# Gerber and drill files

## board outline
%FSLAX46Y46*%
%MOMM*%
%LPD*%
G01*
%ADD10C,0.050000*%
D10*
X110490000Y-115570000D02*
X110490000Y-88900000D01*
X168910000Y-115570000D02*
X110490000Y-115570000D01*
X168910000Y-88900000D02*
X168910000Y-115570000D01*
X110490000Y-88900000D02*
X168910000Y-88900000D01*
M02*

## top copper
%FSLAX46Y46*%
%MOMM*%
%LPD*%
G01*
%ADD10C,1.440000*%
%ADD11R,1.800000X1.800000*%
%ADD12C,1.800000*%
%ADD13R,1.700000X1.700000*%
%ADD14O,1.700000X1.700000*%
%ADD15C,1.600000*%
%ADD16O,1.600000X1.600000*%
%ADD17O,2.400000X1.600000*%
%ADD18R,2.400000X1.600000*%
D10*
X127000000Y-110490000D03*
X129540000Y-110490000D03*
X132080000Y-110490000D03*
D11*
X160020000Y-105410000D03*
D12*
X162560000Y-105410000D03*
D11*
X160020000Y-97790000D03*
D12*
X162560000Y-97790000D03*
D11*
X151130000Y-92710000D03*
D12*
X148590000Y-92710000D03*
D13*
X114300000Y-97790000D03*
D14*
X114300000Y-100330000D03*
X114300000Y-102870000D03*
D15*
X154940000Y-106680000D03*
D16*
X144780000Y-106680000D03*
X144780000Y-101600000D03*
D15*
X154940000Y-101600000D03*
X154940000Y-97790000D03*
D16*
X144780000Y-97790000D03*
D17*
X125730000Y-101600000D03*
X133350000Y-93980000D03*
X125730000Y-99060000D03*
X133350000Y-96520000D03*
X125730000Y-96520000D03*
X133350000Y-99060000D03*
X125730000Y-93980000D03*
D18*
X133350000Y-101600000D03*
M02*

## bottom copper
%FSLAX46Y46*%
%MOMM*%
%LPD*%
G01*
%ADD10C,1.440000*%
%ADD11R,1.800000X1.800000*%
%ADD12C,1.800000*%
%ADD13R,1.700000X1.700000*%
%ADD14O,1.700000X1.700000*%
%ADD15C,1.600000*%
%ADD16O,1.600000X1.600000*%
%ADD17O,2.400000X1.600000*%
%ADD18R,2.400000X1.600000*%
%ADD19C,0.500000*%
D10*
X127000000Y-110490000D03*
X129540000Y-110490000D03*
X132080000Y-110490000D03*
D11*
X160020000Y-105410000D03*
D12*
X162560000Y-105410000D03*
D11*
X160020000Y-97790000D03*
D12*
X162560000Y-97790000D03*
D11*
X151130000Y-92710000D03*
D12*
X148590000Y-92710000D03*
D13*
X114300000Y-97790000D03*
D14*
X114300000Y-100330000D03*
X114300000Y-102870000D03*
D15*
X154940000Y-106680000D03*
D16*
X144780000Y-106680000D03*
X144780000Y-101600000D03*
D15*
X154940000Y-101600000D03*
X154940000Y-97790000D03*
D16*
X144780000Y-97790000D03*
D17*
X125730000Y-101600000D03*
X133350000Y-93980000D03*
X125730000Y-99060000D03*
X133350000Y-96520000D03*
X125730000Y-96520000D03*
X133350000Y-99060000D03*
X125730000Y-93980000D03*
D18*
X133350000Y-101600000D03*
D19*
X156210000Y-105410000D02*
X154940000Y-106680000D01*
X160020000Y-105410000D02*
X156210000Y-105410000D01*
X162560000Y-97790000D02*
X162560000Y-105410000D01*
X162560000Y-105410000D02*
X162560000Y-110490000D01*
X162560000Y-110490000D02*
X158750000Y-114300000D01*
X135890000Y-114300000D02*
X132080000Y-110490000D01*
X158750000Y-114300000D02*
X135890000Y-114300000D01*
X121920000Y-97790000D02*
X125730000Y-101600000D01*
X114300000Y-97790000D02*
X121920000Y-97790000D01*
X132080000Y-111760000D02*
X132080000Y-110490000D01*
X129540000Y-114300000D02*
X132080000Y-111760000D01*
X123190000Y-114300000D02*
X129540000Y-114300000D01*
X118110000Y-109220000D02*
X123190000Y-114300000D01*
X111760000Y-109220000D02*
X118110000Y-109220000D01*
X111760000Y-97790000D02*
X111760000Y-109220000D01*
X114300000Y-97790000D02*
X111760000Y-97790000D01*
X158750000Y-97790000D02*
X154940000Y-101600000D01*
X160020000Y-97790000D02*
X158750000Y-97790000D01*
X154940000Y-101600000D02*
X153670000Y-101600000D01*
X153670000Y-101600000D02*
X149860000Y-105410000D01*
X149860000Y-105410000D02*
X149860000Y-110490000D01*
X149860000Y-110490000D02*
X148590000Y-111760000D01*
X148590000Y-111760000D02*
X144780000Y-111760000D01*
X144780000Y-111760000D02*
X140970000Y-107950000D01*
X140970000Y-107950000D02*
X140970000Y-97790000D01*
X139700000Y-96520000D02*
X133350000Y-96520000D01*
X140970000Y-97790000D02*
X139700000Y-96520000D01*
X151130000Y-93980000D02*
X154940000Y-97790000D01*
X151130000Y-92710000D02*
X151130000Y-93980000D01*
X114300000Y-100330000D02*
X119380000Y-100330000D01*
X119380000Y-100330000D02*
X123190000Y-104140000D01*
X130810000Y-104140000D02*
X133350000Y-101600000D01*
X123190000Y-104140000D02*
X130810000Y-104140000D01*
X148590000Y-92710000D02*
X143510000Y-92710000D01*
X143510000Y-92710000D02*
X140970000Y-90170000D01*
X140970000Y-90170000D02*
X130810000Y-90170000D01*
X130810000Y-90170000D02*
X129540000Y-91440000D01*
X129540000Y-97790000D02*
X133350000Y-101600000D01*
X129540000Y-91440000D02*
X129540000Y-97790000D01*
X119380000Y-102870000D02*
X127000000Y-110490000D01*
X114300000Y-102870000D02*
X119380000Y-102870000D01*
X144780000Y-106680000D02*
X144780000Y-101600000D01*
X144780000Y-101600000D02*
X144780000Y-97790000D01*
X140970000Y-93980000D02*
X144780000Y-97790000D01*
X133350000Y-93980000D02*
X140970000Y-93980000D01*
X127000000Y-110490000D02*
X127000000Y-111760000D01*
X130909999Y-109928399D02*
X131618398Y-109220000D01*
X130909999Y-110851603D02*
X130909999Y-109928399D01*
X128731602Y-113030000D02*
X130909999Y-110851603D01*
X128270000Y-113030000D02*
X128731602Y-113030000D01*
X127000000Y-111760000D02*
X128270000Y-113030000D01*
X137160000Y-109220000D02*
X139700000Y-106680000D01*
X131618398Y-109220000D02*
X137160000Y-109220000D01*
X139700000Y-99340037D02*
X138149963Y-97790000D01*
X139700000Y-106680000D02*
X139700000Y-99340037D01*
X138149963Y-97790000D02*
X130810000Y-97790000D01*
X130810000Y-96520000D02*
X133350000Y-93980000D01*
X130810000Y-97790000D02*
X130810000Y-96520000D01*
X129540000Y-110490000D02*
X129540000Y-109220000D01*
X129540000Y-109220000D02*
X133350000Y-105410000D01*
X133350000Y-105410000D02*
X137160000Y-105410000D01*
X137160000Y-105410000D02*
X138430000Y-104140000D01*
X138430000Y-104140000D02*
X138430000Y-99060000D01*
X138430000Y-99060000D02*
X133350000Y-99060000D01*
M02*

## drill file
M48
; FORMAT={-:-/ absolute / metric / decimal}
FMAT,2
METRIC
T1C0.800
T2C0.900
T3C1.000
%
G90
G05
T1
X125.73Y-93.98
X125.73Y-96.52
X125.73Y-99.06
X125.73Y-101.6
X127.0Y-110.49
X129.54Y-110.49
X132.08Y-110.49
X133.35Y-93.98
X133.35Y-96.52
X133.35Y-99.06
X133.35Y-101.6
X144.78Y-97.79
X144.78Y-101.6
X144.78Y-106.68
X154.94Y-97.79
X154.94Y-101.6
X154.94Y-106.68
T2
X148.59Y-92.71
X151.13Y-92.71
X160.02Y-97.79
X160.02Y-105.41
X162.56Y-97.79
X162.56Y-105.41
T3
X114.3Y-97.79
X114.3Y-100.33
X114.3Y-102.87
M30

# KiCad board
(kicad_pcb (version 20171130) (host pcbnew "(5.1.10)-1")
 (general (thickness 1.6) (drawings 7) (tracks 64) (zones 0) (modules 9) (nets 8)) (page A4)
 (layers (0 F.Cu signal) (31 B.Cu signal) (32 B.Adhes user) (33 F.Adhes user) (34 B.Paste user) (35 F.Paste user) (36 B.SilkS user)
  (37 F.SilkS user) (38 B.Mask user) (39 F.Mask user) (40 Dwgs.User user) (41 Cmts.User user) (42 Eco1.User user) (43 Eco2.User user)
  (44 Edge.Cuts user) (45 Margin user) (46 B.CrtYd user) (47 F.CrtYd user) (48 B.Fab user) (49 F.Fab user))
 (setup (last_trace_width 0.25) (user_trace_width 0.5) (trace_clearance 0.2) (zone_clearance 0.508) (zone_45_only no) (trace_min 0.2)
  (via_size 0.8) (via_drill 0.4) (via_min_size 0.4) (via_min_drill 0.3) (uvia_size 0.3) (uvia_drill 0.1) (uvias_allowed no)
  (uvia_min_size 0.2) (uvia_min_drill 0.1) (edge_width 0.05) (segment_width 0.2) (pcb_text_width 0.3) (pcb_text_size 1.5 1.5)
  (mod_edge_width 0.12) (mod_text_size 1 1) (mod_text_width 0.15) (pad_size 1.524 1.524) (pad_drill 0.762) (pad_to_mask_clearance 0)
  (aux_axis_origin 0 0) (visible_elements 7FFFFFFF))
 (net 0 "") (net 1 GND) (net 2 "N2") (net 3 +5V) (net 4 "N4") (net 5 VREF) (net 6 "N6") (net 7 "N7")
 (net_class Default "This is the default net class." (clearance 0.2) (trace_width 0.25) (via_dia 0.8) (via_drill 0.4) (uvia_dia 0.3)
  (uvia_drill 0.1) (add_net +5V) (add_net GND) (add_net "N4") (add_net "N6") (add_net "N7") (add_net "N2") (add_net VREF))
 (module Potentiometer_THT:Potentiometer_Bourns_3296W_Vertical (layer F.Cu) (at 132.08 110.49)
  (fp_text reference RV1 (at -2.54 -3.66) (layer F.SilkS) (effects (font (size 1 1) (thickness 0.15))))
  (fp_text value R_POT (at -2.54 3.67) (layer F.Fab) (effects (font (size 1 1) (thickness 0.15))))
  (pad 3 thru_hole circle (at -5.08 0) (size 1.44 1.44) (drill 0.8) (layers *.Cu *.Mask) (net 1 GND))
  (pad 2 thru_hole circle (at -2.54 0) (size 1.44 1.44) (drill 0.8) (layers *.Cu *.Mask) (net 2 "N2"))
  (pad 1 thru_hole circle (at 0 0) (size 1.44 1.44) (drill 0.8) (layers *.Cu *.Mask) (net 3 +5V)))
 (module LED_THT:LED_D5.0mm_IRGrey (layer F.Cu) (at 160.02 105.41)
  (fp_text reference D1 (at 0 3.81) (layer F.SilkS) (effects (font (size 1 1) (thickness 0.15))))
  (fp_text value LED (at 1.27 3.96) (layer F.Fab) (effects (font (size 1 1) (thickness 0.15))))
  (pad 1 thru_hole rect (at 0 0) (size 1.8 1.8) (drill 0.9) (layers *.Cu *.Mask) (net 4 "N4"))
  (pad 2 thru_hole circle (at 2.54 0) (size 1.8 1.8) (drill 0.9) (layers *.Cu *.Mask) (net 3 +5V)))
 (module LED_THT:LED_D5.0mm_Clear (layer F.Cu) (at 160.02 97.79)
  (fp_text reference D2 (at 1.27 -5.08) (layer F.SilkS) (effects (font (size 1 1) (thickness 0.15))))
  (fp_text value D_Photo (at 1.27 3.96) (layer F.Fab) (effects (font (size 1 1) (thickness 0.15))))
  (pad 1 thru_hole rect (at 0 0) (size 1.8 1.8) (drill 0.9) (layers *.Cu *.Mask) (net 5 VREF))
  (pad 2 thru_hole circle (at 2.54 0) (size 1.8 1.8) (drill 0.9) (layers *.Cu *.Mask) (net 3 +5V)))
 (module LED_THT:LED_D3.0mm (layer F.Cu) (at 151.13 92.71 180)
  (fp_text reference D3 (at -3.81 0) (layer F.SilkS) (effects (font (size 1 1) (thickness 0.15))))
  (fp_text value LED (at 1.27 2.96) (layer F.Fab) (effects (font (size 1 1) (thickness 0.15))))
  (pad 1 thru_hole rect (at 0 0 180) (size 1.8 1.8) (drill 0.9) (layers *.Cu *.Mask) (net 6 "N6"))
  (pad 2 thru_hole circle (at 2.54 0 180) (size 1.8 1.8) (drill 0.9) (layers *.Cu *.Mask) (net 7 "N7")))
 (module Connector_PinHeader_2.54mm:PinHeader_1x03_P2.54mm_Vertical (layer F.Cu) (at 114.3 97.79)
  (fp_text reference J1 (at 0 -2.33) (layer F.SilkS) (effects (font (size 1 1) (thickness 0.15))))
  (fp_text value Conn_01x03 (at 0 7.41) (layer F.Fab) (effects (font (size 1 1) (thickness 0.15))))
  (pad 1 thru_hole rect (at 0 0) (size 1.7 1.7) (drill 1) (layers *.Cu *.Mask) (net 3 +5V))
  (pad 2 thru_hole oval (at 0 2.54) (size 1.7 1.7) (drill 1) (layers *.Cu *.Mask) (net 7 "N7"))
  (pad 3 thru_hole oval (at 0 5.08) (size 1.7 1.7) (drill 1) (layers *.Cu *.Mask) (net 1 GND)))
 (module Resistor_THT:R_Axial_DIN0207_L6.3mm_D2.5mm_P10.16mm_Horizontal (layer F.Cu) (at 154.94 106.68 180)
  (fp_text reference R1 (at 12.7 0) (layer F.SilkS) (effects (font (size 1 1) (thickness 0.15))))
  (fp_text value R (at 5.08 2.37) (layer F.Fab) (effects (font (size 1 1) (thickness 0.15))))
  (pad 1 thru_hole circle (at 0 0 180) (size 1.6 1.6) (drill 0.8) (layers *.Cu *.Mask) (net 4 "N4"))
  (pad 2 thru_hole oval (at 10.16 0 180) (size 1.6 1.6) (drill 0.8) (layers *.Cu *.Mask) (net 1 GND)))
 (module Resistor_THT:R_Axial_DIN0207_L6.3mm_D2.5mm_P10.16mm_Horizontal (layer F.Cu) (at 154.94 101.6 180)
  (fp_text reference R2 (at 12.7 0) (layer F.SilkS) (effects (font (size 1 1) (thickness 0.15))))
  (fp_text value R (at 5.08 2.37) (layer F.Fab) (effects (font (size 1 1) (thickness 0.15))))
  (pad 2 thru_hole oval (at 10.16 0 180) (size 1.6 1.6) (drill 0.8) (layers *.Cu *.Mask) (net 1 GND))
  (pad 1 thru_hole circle (at 0 0 180) (size 1.6 1.6) (drill 0.8) (layers *.Cu *.Mask) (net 5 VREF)))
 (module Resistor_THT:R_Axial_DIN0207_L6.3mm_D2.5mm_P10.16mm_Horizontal (layer F.Cu) (at 154.94 97.79 180)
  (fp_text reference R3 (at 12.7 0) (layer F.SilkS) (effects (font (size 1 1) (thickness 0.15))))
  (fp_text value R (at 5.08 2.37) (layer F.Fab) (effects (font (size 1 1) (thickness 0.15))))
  (pad 1 thru_hole circle (at 0 0 180) (size 1.6 1.6) (drill 0.8) (layers *.Cu *.Mask) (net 6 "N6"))
  (pad 2 thru_hole oval (at 10.16 0 180) (size 1.6 1.6) (drill 0.8) (layers *.Cu *.Mask) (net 1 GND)))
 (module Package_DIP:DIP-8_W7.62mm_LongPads (layer F.Cu) (at 133.35 101.6 180)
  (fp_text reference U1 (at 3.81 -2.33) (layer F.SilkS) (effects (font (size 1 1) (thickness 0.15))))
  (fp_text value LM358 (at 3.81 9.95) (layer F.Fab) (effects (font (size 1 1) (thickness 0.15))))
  (pad 8 thru_hole oval (at 7.62 0 180) (size 2.4 1.6) (drill 0.8) (layers *.Cu *.Mask) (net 3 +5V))
  (pad 4 thru_hole oval (at 0 7.62 180) (size 2.4 1.6) (drill 0.8) (layers *.Cu *.Mask) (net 1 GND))
  (pad 7 thru_hole oval (at 7.62 2.54 180) (size 2.4 1.6) (drill 0.8) (layers *.Cu *.Mask))
  (pad 3 thru_hole oval (at 0 5.08 180) (size 2.4 1.6) (drill 0.8) (layers *.Cu *.Mask) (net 5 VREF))
  (pad 6 thru_hole oval (at 7.62 5.08 180) (size 2.4 1.6) (drill 0.8) (layers *.Cu *.Mask))
  (pad 2 thru_hole oval (at 0 2.54 180) (size 2.4 1.6) (drill 0.8) (layers *.Cu *.Mask) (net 2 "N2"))
  (pad 5 thru_hole oval (at 7.62 7.62 180) (size 2.4 1.6) (drill 0.8) (layers *.Cu *.Mask))
  (pad 1 thru_hole rect (at 0 0 180) (size 2.4 1.6) (drill 0.8) (layers *.Cu *.Mask) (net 7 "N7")))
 (gr_line (start 110.49 115.57) (end 110.49 88.9) (layer Edge.Cuts) (width 0.05))
 (gr_line (start 168.91 115.57) (end 110.49 115.57) (layer Edge.Cuts) (width 0.05))
 (gr_line (start 168.91 88.9) (end 168.91 115.57) (layer Edge.Cuts) (width 0.05))
 (gr_line (start 110.49 88.9) (end 168.91 88.9) (layer Edge.Cuts) (width 0.05))
 (segment (start 156.21 105.41) (end 154.94 106.68) (width 0.5) (layer B.Cu) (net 4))
 (segment (start 160.02 105.41) (end 156.21 105.41) (width 0.5) (layer B.Cu) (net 4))
 (segment (start 162.56 97.79) (end 162.56 105.41) (width 0.5) (layer B.Cu) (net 3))
 (segment (start 162.56 105.41) (end 162.56 110.49) (width 0.5) (layer B.Cu) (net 3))
 (segment (start 162.56 110.49) (end 158.75 114.3) (width 0.5) (layer B.Cu) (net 3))
 (segment (start 135.89 114.3) (end 132.08 110.49) (width 0.5) (layer B.Cu) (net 3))
 (segment (start 158.75 114.3) (end 135.89 114.3) (width 0.5) (layer B.Cu) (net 3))
 (segment (start 121.92 97.79) (end 125.73 101.6) (width 0.5) (layer B.Cu) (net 3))
 (segment (start 114.3 97.79) (end 121.92 97.79) (width 0.5) (layer B.Cu) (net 3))
 (segment (start 132.08 111.76) (end 132.08 110.49) (width 0.5) (layer B.Cu) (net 3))
 (segment (start 129.54 114.3) (end 132.08 111.76) (width 0.5) (layer B.Cu) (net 3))
 (segment (start 123.19 114.3) (end 129.54 114.3) (width 0.5) (layer B.Cu) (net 3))
 (segment (start 118.11 109.22) (end 123.19 114.3) (width 0.5) (layer B.Cu) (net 3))
 (segment (start 111.76 109.22) (end 118.11 109.22) (width 0.5) (layer B.Cu) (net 3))
 (segment (start 111.76 97.79) (end 111.76 109.22) (width 0.5) (layer B.Cu) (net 3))
 (segment (start 114.3 97.79) (end 111.76 97.79) (width 0.5) (layer B.Cu) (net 3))
 (segment (start 158.75 97.79) (end 154.94 101.6) (width 0.5) (layer B.Cu) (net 5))
 (segment (start 160.02 97.79) (end 158.75 97.79) (width 0.5) (layer B.Cu) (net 5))
 (segment (start 154.94 101.6) (end 153.67 101.6) (width 0.5) (layer B.Cu) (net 5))
 (segment (start 153.67 101.6) (end 149.86 105.41) (width 0.5) (layer B.Cu) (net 5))
 (segment (start 149.86 105.41) (end 149.86 110.49) (width 0.5) (layer B.Cu) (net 5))
 (segment (start 149.86 110.49) (end 148.59 111.76) (width 0.5) (layer B.Cu) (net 5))
 (segment (start 148.59 111.76) (end 144.78 111.76) (width 0.5) (layer B.Cu) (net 5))
 (segment (start 144.78 111.76) (end 140.97 107.95) (width 0.5) (layer B.Cu) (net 5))
 (segment (start 140.97 107.95) (end 140.97 97.79) (width 0.5) (layer B.Cu) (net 5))
 (segment (start 139.7 96.52) (end 133.35 96.52) (width 0.5) (layer B.Cu) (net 5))
 (segment (start 140.97 97.79) (end 139.7 96.52) (width 0.5) (layer B.Cu) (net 5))
 (segment (start 151.13 93.98) (end 154.94 97.79) (width 0.5) (layer B.Cu) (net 6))
 (segment (start 151.13 92.71) (end 151.13 93.98) (width 0.5) (layer B.Cu) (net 6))
 (segment (start 114.3 100.33) (end 119.38 100.33) (width 0.5) (layer B.Cu) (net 7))
 (segment (start 119.38 100.33) (end 123.19 104.14) (width 0.5) (layer B.Cu) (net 7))
 (segment (start 130.81 104.14) (end 133.35 101.6) (width 0.5) (layer B.Cu) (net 7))
 (segment (start 123.19 104.14) (end 130.81 104.14) (width 0.5) (layer B.Cu) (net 7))
 (segment (start 148.59 92.71) (end 143.51 92.71) (width 0.5) (layer B.Cu) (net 7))
 (segment (start 143.51 92.71) (end 140.97 90.17) (width 0.5) (layer B.Cu) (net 7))
 (segment (start 140.97 90.17) (end 130.81 90.17) (width 0.5) (layer B.Cu) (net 7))
 (segment (start 130.81 90.17) (end 129.54 91.44) (width 0.5) (layer B.Cu) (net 7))
 (segment (start 129.54 97.79) (end 133.35 101.6) (width 0.5) (layer B.Cu) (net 7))
 (segment (start 129.54 91.44) (end 129.54 97.79) (width 0.5) (layer B.Cu) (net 7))
 (segment (start 119.38 102.87) (end 127 110.49) (width 0.5) (layer B.Cu) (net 1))
 (segment (start 114.3 102.87) (end 119.38 102.87) (width 0.5) (layer B.Cu) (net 1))
 (segment (start 144.78 106.68) (end 144.78 101.6) (width 0.5) (layer B.Cu) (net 1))
 (segment (start 144.78 101.6) (end 144.78 97.79) (width 0.5) (layer B.Cu) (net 1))
 (segment (start 140.97 93.98) (end 144.78 97.79) (width 0.5) (layer B.Cu) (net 1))
 (segment (start 133.35 93.98) (end 140.97 93.98) (width 0.5) (layer B.Cu) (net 1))
 (segment (start 127 110.49) (end 127 111.76) (width 0.5) (layer B.Cu) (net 1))
 (segment (start 130.909999 109.928399) (end 131.618398 109.22) (width 0.5) (layer B.Cu) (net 1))
 (segment (start 130.909999 110.851603) (end 130.909999 109.928399) (width 0.5) (layer B.Cu) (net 1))
 (segment (start 128.731602 113.03) (end 130.909999 110.851603) (width 0.5) (layer B.Cu) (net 1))
 (segment (start 128.27 113.03) (end 128.731602 113.03) (width 0.5) (layer B.Cu) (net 1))
 (segment (start 127 111.76) (end 128.27 113.03) (width 0.5) (layer B.Cu) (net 1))
 (segment (start 137.16 109.22) (end 139.7 106.68) (width 0.5) (layer B.Cu) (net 1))
 (segment (start 131.618398 109.22) (end 137.16 109.22) (width 0.5) (layer B.Cu) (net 1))
 (segment (start 139.7 99.340037) (end 138.149963 97.79) (width 0.5) (layer B.Cu) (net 1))
 (segment (start 139.7 106.68) (end 139.7 99.340037) (width 0.5) (layer B.Cu) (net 1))
 (segment (start 138.149963 97.79) (end 130.81 97.79) (width 0.5) (layer B.Cu) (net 1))
 (segment (start 130.81 96.52) (end 133.35 93.98) (width 0.5) (layer B.Cu) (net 1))
 (segment (start 130.81 97.79) (end 130.81 96.52) (width 0.5) (layer B.Cu) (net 1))
 (segment (start 129.54 110.49) (end 129.54 109.22) (width 0.5) (layer B.Cu) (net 2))
 (segment (start 129.54 109.22) (end 133.35 105.41) (width 0.5) (layer B.Cu) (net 2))
 (segment (start 133.35 105.41) (end 137.16 105.41) (width 0.5) (layer B.Cu) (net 2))
 (segment (start 137.16 105.41) (end 138.43 104.14) (width 0.5) (layer B.Cu) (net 2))
 (segment (start 138.43 104.14) (end 138.43 99.06) (width 0.5) (layer B.Cu) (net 2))
 (segment (start 138.43 99.06) (end 133.35 99.06) (width 0.5) (layer B.Cu) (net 2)))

